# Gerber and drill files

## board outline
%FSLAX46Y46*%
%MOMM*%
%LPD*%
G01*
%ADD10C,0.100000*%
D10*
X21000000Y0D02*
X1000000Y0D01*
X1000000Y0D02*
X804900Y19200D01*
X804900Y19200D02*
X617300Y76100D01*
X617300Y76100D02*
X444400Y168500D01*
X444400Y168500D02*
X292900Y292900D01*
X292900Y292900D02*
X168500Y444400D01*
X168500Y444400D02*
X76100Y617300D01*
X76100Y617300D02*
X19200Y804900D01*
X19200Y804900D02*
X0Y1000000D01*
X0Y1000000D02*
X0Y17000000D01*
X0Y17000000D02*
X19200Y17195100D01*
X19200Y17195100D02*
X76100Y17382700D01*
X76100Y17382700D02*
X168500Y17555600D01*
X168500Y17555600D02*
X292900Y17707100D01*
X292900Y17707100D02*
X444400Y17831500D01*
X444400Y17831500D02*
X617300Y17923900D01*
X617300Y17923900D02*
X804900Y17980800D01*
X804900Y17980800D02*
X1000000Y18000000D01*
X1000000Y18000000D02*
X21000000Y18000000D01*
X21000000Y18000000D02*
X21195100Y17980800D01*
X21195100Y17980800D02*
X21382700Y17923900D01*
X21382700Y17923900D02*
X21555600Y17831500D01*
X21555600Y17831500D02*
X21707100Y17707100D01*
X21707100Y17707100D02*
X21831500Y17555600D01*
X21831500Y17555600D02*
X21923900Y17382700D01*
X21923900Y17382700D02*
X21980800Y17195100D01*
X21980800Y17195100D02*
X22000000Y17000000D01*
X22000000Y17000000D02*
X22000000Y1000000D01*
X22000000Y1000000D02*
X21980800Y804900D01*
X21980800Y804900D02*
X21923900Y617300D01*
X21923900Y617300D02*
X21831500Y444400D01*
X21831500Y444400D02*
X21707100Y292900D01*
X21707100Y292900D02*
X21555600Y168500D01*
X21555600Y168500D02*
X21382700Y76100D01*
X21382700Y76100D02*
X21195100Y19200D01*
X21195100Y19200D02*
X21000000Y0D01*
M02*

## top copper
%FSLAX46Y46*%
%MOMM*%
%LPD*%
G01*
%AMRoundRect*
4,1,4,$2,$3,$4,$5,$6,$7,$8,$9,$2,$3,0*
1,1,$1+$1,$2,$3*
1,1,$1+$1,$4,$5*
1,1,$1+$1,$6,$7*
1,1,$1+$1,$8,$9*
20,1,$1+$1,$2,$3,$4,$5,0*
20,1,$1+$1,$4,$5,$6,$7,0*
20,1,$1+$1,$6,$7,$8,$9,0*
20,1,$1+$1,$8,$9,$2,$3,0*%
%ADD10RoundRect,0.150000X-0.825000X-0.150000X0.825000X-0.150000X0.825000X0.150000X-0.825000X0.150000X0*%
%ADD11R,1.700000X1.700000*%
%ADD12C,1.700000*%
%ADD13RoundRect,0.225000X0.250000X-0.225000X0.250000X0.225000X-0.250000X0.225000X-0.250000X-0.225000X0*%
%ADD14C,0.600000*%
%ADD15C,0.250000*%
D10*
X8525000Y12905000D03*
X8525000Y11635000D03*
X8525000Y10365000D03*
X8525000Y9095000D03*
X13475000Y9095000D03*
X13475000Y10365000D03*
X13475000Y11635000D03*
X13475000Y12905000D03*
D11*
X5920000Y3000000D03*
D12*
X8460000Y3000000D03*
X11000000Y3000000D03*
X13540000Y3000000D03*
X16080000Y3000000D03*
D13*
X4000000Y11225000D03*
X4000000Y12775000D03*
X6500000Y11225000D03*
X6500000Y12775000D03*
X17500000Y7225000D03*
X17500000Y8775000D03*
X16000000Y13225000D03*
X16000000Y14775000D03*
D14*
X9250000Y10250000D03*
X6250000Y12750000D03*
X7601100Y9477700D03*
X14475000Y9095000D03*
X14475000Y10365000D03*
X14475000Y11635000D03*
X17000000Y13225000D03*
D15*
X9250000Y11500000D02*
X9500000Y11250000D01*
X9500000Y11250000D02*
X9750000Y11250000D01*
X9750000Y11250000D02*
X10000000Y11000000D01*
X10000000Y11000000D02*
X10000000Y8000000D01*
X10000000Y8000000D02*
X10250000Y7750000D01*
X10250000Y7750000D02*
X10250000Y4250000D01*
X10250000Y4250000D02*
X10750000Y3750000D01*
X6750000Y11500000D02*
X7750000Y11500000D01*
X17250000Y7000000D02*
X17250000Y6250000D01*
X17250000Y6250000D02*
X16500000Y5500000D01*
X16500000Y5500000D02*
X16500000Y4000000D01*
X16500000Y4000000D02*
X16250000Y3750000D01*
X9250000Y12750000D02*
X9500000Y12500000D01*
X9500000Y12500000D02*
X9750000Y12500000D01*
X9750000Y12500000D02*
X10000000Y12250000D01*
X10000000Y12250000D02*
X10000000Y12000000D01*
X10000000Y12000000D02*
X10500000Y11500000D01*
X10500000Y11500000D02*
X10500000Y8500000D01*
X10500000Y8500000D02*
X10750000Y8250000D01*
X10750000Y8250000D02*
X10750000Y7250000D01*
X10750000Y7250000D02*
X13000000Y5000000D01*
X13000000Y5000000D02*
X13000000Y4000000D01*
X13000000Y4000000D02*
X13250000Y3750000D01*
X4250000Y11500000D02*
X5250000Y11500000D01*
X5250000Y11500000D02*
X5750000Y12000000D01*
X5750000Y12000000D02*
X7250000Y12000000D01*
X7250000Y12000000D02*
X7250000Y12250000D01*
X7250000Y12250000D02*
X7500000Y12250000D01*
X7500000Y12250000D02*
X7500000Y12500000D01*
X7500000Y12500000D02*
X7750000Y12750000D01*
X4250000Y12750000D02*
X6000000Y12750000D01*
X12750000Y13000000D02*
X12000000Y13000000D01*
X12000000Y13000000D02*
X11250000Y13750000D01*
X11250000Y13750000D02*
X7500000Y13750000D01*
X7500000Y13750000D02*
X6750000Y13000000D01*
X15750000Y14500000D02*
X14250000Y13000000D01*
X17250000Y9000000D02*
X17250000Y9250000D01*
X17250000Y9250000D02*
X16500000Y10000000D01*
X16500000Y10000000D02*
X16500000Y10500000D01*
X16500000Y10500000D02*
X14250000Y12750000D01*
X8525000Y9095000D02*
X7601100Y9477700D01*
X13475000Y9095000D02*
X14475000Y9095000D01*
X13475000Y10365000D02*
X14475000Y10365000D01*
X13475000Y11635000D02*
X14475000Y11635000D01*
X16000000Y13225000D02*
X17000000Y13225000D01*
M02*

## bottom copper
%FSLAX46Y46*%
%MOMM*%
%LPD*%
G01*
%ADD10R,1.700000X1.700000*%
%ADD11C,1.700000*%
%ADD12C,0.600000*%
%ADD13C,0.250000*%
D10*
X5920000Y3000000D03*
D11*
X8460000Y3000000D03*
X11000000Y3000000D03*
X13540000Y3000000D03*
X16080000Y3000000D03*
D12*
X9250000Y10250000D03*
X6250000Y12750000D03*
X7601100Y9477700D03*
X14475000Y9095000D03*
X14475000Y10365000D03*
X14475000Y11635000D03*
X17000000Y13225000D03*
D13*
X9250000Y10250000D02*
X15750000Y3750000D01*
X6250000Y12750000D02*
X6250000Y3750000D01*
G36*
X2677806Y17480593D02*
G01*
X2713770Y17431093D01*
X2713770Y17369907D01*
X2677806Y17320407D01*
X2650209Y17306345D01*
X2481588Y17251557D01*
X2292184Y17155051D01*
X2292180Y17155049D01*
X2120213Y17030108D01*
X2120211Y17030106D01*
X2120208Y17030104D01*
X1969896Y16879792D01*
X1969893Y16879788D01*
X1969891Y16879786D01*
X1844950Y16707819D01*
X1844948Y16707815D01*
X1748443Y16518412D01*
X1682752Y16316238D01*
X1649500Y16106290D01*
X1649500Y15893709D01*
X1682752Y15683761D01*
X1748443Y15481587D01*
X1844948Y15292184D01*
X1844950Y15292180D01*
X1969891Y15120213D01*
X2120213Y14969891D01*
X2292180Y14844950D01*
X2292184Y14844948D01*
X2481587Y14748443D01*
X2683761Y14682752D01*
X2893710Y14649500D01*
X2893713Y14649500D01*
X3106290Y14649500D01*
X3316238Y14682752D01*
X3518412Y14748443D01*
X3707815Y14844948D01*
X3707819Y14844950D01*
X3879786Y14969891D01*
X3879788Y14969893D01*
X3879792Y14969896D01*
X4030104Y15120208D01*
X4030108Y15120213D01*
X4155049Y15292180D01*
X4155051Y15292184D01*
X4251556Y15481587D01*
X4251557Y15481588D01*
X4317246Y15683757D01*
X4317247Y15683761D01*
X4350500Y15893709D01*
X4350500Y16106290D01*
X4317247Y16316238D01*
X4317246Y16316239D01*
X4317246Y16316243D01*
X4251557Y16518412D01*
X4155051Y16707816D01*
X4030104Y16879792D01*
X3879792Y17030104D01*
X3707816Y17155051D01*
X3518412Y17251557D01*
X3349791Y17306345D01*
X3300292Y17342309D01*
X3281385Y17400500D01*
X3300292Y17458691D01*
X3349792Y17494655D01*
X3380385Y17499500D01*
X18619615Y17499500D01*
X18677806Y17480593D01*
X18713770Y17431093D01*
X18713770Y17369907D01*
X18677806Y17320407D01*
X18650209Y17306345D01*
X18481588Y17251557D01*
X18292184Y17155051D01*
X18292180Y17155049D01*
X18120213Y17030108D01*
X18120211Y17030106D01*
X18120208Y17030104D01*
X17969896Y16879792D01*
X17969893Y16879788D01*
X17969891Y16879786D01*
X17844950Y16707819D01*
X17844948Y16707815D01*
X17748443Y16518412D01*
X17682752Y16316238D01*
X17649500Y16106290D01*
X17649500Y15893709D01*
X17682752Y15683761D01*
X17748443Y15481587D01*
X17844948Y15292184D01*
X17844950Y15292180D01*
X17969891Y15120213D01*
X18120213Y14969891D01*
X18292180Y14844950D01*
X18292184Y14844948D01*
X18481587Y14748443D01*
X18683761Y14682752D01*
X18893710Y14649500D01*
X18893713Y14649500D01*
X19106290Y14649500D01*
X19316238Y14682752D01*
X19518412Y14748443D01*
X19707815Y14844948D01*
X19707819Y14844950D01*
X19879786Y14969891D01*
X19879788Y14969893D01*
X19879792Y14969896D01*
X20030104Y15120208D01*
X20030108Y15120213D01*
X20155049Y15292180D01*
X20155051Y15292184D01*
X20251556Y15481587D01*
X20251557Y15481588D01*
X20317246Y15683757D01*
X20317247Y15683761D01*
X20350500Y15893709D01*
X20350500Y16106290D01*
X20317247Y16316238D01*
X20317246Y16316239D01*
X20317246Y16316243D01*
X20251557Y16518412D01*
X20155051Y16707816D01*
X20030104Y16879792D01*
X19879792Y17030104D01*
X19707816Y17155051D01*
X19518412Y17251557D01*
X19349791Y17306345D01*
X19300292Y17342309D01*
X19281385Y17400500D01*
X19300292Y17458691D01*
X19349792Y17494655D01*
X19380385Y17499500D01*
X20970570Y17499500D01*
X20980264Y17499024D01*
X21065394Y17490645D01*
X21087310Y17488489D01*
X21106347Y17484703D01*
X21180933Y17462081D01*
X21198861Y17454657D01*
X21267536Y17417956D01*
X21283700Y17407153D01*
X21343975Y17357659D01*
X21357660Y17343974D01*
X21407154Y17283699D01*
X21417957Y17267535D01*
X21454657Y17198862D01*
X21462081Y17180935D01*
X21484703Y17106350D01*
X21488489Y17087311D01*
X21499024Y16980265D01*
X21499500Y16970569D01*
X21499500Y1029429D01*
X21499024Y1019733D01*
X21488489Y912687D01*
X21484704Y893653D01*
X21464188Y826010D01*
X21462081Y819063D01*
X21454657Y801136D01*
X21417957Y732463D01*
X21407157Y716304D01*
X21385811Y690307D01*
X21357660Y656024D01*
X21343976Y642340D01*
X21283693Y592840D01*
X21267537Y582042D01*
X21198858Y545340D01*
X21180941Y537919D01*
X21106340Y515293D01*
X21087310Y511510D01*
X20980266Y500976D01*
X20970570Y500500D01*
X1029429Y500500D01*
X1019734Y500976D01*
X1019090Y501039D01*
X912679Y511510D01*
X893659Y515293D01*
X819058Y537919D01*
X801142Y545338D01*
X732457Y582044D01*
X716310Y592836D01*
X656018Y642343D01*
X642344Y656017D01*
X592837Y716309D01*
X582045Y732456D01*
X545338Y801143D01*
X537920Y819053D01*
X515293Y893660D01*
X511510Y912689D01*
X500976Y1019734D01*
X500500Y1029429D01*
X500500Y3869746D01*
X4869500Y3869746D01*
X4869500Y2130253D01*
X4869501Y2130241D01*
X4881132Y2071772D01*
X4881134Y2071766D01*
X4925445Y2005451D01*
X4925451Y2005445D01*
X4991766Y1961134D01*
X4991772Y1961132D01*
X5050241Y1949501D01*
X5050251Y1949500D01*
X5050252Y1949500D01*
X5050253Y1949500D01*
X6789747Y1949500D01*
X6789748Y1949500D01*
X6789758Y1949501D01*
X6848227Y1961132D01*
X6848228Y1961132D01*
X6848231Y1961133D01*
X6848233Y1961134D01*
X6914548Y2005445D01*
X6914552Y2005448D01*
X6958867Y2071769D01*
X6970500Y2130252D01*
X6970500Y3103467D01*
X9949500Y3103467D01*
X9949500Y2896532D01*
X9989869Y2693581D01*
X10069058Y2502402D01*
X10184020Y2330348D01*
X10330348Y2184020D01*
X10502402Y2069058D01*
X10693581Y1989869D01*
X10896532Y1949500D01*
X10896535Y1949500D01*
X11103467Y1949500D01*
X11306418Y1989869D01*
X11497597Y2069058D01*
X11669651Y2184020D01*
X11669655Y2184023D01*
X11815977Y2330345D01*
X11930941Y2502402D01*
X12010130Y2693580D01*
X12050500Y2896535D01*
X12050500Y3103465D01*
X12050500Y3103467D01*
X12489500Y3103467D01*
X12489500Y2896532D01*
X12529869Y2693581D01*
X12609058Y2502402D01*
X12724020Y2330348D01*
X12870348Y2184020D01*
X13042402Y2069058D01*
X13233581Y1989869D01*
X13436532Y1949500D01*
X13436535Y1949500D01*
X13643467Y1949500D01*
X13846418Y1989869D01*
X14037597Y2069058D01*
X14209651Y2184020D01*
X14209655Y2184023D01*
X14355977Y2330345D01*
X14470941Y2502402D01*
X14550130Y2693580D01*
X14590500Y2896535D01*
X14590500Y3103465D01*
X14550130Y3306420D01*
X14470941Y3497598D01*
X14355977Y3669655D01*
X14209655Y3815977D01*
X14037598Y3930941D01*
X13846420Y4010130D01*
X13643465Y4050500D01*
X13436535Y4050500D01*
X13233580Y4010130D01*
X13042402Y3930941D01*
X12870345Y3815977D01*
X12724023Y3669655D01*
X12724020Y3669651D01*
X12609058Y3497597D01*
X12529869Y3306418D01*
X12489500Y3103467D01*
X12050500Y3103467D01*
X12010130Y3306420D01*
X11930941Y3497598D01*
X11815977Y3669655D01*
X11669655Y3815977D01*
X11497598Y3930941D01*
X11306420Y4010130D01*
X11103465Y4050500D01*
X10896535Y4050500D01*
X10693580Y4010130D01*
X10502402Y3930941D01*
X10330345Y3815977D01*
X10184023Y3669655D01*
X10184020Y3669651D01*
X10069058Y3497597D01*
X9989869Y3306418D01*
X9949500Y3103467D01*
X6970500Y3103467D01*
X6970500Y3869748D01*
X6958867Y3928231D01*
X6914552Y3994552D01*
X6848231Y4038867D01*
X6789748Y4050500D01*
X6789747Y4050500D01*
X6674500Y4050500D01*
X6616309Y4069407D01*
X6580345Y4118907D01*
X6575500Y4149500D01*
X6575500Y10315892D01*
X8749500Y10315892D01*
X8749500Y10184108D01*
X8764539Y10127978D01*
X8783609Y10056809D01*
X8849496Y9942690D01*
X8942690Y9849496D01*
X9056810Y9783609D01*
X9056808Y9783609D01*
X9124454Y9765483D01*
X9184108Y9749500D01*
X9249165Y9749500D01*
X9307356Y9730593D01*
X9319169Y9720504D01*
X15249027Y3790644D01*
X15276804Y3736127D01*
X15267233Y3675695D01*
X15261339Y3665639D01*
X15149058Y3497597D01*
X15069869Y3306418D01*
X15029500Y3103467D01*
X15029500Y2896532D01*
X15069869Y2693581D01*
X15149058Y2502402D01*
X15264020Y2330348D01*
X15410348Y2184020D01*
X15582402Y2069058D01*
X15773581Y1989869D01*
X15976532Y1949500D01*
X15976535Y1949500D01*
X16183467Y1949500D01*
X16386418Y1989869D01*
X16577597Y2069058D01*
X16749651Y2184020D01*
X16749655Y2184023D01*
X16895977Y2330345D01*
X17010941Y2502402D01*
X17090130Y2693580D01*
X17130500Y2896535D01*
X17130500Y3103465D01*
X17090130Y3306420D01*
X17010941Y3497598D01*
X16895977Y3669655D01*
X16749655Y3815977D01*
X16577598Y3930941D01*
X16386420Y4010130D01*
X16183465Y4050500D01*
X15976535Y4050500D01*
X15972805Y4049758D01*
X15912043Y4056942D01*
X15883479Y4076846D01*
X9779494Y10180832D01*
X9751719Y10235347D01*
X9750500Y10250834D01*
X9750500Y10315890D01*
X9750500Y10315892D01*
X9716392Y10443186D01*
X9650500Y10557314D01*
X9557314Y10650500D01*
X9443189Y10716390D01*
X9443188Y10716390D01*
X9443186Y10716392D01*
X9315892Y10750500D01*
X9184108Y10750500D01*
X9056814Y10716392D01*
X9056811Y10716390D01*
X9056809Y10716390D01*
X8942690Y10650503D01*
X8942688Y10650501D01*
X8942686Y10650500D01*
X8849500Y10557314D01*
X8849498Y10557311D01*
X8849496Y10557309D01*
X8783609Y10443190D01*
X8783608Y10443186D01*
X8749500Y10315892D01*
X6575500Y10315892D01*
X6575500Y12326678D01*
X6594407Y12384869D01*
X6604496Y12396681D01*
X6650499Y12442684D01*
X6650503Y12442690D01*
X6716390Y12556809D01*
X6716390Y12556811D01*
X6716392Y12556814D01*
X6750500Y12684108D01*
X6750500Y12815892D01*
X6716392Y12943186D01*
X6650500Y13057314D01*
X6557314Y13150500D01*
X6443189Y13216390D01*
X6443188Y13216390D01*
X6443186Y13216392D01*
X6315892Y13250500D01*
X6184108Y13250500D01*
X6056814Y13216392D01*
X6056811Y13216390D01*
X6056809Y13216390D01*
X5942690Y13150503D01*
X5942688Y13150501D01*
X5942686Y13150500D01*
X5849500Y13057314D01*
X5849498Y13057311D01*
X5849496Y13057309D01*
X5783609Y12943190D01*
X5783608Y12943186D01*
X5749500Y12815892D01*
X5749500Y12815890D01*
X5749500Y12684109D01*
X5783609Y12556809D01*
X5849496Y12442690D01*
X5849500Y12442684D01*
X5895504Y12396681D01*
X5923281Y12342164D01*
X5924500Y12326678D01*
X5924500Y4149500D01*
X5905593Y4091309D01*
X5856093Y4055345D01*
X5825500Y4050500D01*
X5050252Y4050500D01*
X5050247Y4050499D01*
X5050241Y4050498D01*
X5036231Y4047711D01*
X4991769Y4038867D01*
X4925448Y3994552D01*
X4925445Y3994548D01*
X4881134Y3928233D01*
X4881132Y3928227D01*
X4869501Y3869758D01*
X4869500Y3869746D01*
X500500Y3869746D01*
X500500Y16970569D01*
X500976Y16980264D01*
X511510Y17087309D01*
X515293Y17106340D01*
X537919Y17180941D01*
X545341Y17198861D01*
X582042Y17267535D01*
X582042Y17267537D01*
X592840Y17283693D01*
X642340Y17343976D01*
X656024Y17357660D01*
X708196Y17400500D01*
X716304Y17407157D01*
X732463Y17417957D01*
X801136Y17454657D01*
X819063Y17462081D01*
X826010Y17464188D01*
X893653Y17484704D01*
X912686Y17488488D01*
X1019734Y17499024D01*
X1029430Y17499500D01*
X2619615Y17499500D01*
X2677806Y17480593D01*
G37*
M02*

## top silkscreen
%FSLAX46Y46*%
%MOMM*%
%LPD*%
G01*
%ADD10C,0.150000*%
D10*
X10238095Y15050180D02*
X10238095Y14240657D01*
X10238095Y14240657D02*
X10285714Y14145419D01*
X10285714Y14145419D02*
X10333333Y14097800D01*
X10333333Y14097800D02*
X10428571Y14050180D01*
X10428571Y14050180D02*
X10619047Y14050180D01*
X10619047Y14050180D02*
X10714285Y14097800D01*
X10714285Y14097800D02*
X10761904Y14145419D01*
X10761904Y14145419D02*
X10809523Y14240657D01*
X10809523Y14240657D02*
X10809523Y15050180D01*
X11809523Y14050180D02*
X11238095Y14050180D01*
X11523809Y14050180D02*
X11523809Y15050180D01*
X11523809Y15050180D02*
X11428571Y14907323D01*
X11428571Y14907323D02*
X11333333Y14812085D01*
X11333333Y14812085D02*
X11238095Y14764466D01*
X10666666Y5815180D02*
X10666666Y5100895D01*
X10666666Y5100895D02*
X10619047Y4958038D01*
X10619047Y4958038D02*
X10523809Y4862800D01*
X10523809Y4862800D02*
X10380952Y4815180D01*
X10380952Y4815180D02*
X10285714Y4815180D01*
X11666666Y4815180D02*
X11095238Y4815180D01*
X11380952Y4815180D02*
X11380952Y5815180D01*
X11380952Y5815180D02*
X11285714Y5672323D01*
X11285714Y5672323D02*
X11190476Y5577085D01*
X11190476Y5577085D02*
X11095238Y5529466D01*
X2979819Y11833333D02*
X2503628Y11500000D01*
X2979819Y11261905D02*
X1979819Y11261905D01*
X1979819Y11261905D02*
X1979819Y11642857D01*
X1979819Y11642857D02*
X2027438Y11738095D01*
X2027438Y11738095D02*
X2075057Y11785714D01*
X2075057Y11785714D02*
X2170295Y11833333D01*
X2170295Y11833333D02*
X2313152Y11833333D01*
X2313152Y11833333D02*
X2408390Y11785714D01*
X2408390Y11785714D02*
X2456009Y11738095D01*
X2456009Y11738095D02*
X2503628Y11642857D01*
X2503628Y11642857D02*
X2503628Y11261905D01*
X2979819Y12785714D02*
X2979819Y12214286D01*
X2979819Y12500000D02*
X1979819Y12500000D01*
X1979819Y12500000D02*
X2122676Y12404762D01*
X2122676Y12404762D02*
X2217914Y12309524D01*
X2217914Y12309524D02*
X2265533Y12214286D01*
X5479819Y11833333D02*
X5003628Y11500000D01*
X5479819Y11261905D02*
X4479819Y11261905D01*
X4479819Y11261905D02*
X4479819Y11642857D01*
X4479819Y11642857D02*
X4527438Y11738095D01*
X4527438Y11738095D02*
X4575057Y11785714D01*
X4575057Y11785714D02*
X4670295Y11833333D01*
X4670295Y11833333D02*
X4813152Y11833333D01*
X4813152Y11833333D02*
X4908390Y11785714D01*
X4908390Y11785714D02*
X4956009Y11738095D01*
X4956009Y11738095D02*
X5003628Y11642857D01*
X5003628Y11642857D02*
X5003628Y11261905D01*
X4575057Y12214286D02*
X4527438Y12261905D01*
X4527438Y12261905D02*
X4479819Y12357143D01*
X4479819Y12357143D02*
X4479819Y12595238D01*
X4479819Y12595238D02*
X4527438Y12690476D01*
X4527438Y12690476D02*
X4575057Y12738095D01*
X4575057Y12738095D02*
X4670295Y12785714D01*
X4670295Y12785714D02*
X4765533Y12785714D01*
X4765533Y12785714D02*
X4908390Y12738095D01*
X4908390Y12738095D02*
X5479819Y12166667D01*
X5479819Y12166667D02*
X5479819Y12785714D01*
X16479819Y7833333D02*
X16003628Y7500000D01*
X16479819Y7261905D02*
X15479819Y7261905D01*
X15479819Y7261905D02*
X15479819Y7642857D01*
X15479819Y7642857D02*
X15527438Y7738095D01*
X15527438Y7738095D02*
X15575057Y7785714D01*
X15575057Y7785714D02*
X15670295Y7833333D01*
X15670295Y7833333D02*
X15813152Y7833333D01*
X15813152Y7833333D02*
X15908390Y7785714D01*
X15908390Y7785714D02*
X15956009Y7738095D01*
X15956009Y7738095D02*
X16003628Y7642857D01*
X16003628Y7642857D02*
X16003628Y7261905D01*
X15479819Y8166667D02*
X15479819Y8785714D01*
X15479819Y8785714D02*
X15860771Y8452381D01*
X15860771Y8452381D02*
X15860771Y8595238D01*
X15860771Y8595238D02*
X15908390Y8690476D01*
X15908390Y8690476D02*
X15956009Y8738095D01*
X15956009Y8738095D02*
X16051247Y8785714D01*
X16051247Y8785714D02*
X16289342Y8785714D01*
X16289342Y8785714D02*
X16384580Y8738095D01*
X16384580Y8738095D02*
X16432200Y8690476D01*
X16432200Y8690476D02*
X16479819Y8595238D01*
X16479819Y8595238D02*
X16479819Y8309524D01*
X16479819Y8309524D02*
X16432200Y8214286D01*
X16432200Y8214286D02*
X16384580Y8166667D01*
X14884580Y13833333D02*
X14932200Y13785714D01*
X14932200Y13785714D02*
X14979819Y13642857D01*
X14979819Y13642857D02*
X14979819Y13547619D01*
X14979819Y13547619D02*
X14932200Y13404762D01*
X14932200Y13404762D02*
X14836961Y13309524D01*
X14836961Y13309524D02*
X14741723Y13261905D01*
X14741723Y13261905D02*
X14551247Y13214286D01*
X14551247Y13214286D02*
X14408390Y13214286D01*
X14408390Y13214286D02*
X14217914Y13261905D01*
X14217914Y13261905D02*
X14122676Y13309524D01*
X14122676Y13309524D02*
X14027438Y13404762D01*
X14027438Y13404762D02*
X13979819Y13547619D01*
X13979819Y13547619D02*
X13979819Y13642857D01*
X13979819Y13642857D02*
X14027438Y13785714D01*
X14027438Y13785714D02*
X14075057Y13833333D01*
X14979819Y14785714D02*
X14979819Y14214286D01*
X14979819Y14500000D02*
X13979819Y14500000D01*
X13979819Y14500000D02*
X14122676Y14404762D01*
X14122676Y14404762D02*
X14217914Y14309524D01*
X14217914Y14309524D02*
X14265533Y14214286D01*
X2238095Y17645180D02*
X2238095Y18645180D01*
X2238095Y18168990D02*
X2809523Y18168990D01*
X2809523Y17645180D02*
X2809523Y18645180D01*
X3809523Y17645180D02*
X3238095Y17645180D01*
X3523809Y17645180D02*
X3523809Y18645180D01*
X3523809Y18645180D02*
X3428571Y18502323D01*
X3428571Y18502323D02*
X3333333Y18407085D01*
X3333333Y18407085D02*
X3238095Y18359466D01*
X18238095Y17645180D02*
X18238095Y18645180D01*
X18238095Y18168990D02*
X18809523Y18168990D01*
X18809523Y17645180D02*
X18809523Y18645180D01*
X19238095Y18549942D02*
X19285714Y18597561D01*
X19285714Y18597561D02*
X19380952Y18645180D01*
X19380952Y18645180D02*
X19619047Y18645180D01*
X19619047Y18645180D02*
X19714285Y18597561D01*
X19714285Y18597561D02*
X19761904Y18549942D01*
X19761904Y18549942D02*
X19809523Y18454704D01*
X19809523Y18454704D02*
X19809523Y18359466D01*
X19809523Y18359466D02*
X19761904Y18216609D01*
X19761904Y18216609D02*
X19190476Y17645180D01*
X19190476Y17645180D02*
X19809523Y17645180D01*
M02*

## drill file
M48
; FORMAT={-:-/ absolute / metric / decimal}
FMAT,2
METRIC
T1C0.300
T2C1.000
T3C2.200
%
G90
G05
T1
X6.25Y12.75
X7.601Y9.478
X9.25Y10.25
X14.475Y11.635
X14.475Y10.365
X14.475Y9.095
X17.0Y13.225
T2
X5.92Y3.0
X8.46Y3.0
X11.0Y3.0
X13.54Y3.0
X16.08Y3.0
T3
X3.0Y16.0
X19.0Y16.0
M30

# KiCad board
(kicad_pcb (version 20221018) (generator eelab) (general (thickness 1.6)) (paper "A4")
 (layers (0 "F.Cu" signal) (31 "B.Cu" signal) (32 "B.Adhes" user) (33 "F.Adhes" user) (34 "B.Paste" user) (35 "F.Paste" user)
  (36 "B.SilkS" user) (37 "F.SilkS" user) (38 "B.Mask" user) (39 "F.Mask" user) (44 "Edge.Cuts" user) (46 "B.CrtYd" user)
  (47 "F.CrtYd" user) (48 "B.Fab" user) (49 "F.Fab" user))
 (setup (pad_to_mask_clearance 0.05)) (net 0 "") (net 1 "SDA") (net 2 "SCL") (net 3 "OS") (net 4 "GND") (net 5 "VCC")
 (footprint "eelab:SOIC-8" (layer "F.Cu") (at 11.0000 -11.0000 0)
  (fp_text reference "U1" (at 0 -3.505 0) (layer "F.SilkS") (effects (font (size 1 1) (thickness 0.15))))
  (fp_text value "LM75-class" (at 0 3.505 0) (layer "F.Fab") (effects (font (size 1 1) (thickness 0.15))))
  (pad "1" smd roundrect (at -2.4750 -1.9050 0) (size 1.9500 0.6000) (layers "F.Cu" "F.Paste" "F.Mask") (roundrect_rratio 0.25)
   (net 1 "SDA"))
  (pad "2" smd roundrect (at -2.4750 -0.6350 0) (size 1.9500 0.6000) (layers "F.Cu" "F.Paste" "F.Mask") (roundrect_rratio 0.25)
   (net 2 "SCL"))
  (pad "3" smd roundrect (at -2.4750 0.6350 0) (size 1.9500 0.6000) (layers "F.Cu" "F.Paste" "F.Mask") (roundrect_rratio 0.25) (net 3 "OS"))
  (pad "4" smd roundrect (at -2.4750 1.9050 0) (size 1.9500 0.6000) (layers "F.Cu" "F.Paste" "F.Mask") (roundrect_rratio 0.25) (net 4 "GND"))
  (pad "5" smd roundrect (at 2.4750 1.9050 0) (size 1.9500 0.6000) (layers "F.Cu" "F.Paste" "F.Mask") (roundrect_rratio 0.25) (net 4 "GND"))
  (pad "6" smd roundrect (at 2.4750 0.6350 0) (size 1.9500 0.6000) (layers "F.Cu" "F.Paste" "F.Mask") (roundrect_rratio 0.25) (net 4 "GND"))
  (pad "7" smd roundrect (at 2.4750 -0.6350 0) (size 1.9500 0.6000) (layers "F.Cu" "F.Paste" "F.Mask") (roundrect_rratio 0.25) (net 4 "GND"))
  (pad "8" smd roundrect (at 2.4750 -1.9050 0) (size 1.9500 0.6000) (layers "F.Cu" "F.Paste" "F.Mask") (roundrect_rratio 0.25) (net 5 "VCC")))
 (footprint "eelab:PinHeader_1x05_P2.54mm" (layer "F.Cu") (at 11.0000 -3.0000 0)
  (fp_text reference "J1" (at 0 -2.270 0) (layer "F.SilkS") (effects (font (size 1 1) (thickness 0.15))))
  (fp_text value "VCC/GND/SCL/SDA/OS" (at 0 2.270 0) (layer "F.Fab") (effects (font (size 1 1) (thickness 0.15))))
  (pad "1" thru_hole rect (at -5.0800 -0.0000 0) (size 1.7000 1.7000) (drill 1.0) (layers "*.Cu" "*.Mask") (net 5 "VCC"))
  (pad "2" thru_hole circle (at -2.5400 -0.0000 0) (size 1.7000 1.7000) (drill 1.0) (layers "*.Cu" "*.Mask") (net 4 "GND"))
  (pad "3" thru_hole circle (at 0.0000 -0.0000 0) (size 1.7000 1.7000) (drill 1.0) (layers "*.Cu" "*.Mask") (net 2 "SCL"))
  (pad "4" thru_hole circle (at 2.5400 -0.0000 0) (size 1.7000 1.7000) (drill 1.0) (layers "*.Cu" "*.Mask") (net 1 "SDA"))
  (pad "5" thru_hole circle (at 5.0800 -0.0000 0) (size 1.7000 1.7000) (drill 1.0) (layers "*.Cu" "*.Mask") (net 3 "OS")))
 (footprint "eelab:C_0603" (layer "F.Cu") (at 4.0000 -12.0000 90)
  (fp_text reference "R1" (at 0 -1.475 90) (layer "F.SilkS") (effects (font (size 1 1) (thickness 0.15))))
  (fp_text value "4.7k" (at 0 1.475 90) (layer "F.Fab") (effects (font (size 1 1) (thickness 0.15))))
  (pad "1" smd roundrect (at -0.7750 0.0000 90) (size 0.9000 0.9500) (layers "F.Cu" "F.Paste" "F.Mask") (roundrect_rratio 0.25)
   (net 1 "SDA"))
  (pad "2" smd roundrect (at 0.7750 0.0000 90) (size 0.9000 0.9500) (layers "F.Cu" "F.Paste" "F.Mask") (roundrect_rratio 0.25) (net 5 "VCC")))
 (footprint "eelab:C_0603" (layer "F.Cu") (at 6.5000 -12.0000 90)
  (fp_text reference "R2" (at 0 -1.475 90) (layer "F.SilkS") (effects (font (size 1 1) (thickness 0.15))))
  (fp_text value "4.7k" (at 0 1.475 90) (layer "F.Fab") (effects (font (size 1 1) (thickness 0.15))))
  (pad "1" smd roundrect (at -0.7750 0.0000 90) (size 0.9000 0.9500) (layers "F.Cu" "F.Paste" "F.Mask") (roundrect_rratio 0.25)
   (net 2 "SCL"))
  (pad "2" smd roundrect (at 0.7750 0.0000 90) (size 0.9000 0.9500) (layers "F.Cu" "F.Paste" "F.Mask") (roundrect_rratio 0.25) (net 5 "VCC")))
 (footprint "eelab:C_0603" (layer "F.Cu") (at 17.5000 -8.0000 90)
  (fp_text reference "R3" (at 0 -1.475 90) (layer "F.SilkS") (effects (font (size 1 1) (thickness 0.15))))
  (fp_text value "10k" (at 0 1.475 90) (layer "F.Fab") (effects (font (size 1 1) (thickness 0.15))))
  (pad "1" smd roundrect (at -0.7750 0.0000 90) (size 0.9000 0.9500) (layers "F.Cu" "F.Paste" "F.Mask") (roundrect_rratio 0.25) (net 3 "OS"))
  (pad "2" smd roundrect (at 0.7750 0.0000 90) (size 0.9000 0.9500) (layers "F.Cu" "F.Paste" "F.Mask") (roundrect_rratio 0.25) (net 5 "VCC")))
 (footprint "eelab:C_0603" (layer "F.Cu") (at 16.0000 -14.0000 90)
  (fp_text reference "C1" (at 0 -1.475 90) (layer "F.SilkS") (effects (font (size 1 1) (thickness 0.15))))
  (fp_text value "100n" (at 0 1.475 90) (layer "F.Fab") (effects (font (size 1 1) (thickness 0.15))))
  (pad "1" smd roundrect (at -0.7750 0.0000 90) (size 0.9000 0.9500) (layers "F.Cu" "F.Paste" "F.Mask") (roundrect_rratio 0.25)
   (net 4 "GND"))
  (pad "2" smd roundrect (at 0.7750 0.0000 90) (size 0.9000 0.9500) (layers "F.Cu" "F.Paste" "F.Mask") (roundrect_rratio 0.25) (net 5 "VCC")))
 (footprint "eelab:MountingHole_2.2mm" (layer "F.Cu") (at 3.0000 -16.0000 0)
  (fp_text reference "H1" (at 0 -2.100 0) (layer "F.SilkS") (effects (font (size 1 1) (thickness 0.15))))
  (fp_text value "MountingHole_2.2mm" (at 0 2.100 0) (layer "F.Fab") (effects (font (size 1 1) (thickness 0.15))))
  (pad "" np_thru_hole circle (at 0.0000 0.0000 0) (size 2.2000 2.2000) (drill 2.2) (layers "*.Cu" "*.Mask")))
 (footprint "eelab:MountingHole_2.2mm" (layer "F.Cu") (at 19.0000 -16.0000 0)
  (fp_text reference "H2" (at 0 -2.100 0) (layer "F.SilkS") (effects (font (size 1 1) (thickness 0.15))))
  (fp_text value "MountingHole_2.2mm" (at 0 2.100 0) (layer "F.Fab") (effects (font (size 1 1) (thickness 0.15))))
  (pad "" np_thru_hole circle (at 0.0000 0.0000 0) (size 2.2000 2.2000) (drill 2.2) (layers "*.Cu" "*.Mask")))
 (gr_line (start 21.0000 -0.0000) (end 1.0000 -0.0000) (stroke (width 0.1) (type solid)) (layer "Edge.Cuts"))
 (gr_line (start 1.0000 -0.0000) (end 0.8049 -0.0192) (stroke (width 0.1) (type solid)) (layer "Edge.Cuts"))
 (gr_line (start 0.8049 -0.0192) (end 0.6173 -0.0761) (stroke (width 0.1) (type solid)) (layer "Edge.Cuts"))
 (gr_line (start 0.6173 -0.0761) (end 0.4444 -0.1685) (stroke (width 0.1) (type solid)) (layer "Edge.Cuts"))
 (gr_line (start 0.4444 -0.1685) (end 0.2929 -0.2929) (stroke (width 0.1) (type solid)) (layer "Edge.Cuts"))
 (gr_line (start 0.2929 -0.2929) (end 0.1685 -0.4444) (stroke (width 0.1) (type solid)) (layer "Edge.Cuts"))
 (gr_line (start 0.1685 -0.4444) (end 0.0761 -0.6173) (stroke (width 0.1) (type solid)) (layer "Edge.Cuts"))
 (gr_line (start 0.0761 -0.6173) (end 0.0192 -0.8049) (stroke (width 0.1) (type solid)) (layer "Edge.Cuts"))
 (gr_line (start 0.0192 -0.8049) (end 0.0000 -1.0000) (stroke (width 0.1) (type solid)) (layer "Edge.Cuts"))
 (gr_line (start 0.0000 -1.0000) (end 0.0000 -17.0000) (stroke (width 0.1) (type solid)) (layer "Edge.Cuts"))
 (gr_line (start 0.0000 -17.0000) (end 0.0192 -17.1951) (stroke (width 0.1) (type solid)) (layer "Edge.Cuts"))
 (gr_line (start 0.0192 -17.1951) (end 0.0761 -17.3827) (stroke (width 0.1) (type solid)) (layer "Edge.Cuts"))
 (gr_line (start 0.0761 -17.3827) (end 0.1685 -17.5556) (stroke (width 0.1) (type solid)) (layer "Edge.Cuts"))
 (gr_line (start 0.1685 -17.5556) (end 0.2929 -17.7071) (stroke (width 0.1) (type solid)) (layer "Edge.Cuts"))
 (gr_line (start 0.2929 -17.7071) (end 0.4444 -17.8315) (stroke (width 0.1) (type solid)) (layer "Edge.Cuts"))
 (gr_line (start 0.4444 -17.8315) (end 0.6173 -17.9239) (stroke (width 0.1) (type solid)) (layer "Edge.Cuts"))
 (gr_line (start 0.6173 -17.9239) (end 0.8049 -17.9808) (stroke (width 0.1) (type solid)) (layer "Edge.Cuts"))
 (gr_line (start 0.8049 -17.9808) (end 1.0000 -18.0000) (stroke (width 0.1) (type solid)) (layer "Edge.Cuts"))
 (gr_line (start 1.0000 -18.0000) (end 21.0000 -18.0000) (stroke (width 0.1) (type solid)) (layer "Edge.Cuts"))
 (gr_line (start 21.0000 -18.0000) (end 21.1951 -17.9808) (stroke (width 0.1) (type solid)) (layer "Edge.Cuts"))
 (gr_line (start 21.1951 -17.9808) (end 21.3827 -17.9239) (stroke (width 0.1) (type solid)) (layer "Edge.Cuts"))
 (gr_line (start 21.3827 -17.9239) (end 21.5556 -17.8315) (stroke (width 0.1) (type solid)) (layer "Edge.Cuts"))
 (gr_line (start 21.5556 -17.8315) (end 21.7071 -17.7071) (stroke (width 0.1) (type solid)) (layer "Edge.Cuts"))
 (gr_line (start 21.7071 -17.7071) (end 21.8315 -17.5556) (stroke (width 0.1) (type solid)) (layer "Edge.Cuts"))
 (gr_line (start 21.8315 -17.5556) (end 21.9239 -17.3827) (stroke (width 0.1) (type solid)) (layer "Edge.Cuts"))
 (gr_line (start 21.9239 -17.3827) (end 21.9808 -17.1951) (stroke (width 0.1) (type solid)) (layer "Edge.Cuts"))
 (gr_line (start 21.9808 -17.1951) (end 22.0000 -17.0000) (stroke (width 0.1) (type solid)) (layer "Edge.Cuts"))
 (gr_line (start 22.0000 -17.0000) (end 22.0000 -1.0000) (stroke (width 0.1) (type solid)) (layer "Edge.Cuts"))
 (gr_line (start 22.0000 -1.0000) (end 21.9808 -0.8049) (stroke (width 0.1) (type solid)) (layer "Edge.Cuts"))
 (gr_line (start 21.9808 -0.8049) (end 21.9239 -0.6173) (stroke (width 0.1) (type solid)) (layer "Edge.Cuts"))
 (gr_line (start 21.9239 -0.6173) (end 21.8315 -0.4444) (stroke (width 0.1) (type solid)) (layer "Edge.Cuts"))
 (gr_line (start 21.8315 -0.4444) (end 21.7071 -0.2929) (stroke (width 0.1) (type solid)) (layer "Edge.Cuts"))
 (gr_line (start 21.7071 -0.2929) (end 21.5556 -0.1685) (stroke (width 0.1) (type solid)) (layer "Edge.Cuts"))
 (gr_line (start 21.5556 -0.1685) (end 21.3827 -0.0761) (stroke (width 0.1) (type solid)) (layer "Edge.Cuts"))
 (gr_line (start 21.3827 -0.0761) (end 21.1951 -0.0192) (stroke (width 0.1) (type solid)) (layer "Edge.Cuts"))
 (gr_line (start 21.1951 -0.0192) (end 21.0000 -0.0000) (stroke (width 0.1) (type solid)) (layer "Edge.Cuts"))
 (segment (start 9.2500 -11.5000) (end 9.5000 -11.2500) (width 0.25) (layer "F.Cu") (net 2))
 (segment (start 9.5000 -11.2500) (end 9.7500 -11.2500) (width 0.25) (layer "F.Cu") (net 2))
 (segment (start 9.7500 -11.2500) (end 10.0000 -11.0000) (width 0.25) (layer "F.Cu") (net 2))
 (segment (start 10.0000 -11.0000) (end 10.0000 -8.0000) (width 0.25) (layer "F.Cu") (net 2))
 (segment (start 10.0000 -8.0000) (end 10.2500 -7.7500) (width 0.25) (layer "F.Cu") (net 2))
 (segment (start 10.2500 -7.7500) (end 10.2500 -4.2500) (width 0.25) (layer "F.Cu") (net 2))
 (segment (start 10.2500 -4.2500) (end 10.7500 -3.7500) (width 0.25) (layer "F.Cu") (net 2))
 (segment (start 6.7500 -11.5000) (end 7.7500 -11.5000) (width 0.25) (layer "F.Cu") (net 2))
 (segment (start 17.2500 -7.0000) (end 17.2500 -6.2500) (width 0.25) (layer "F.Cu") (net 3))
 (segment (start 17.2500 -6.2500) (end 16.5000 -5.5000) (width 0.25) (layer "F.Cu") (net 3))
 (segment (start 16.5000 -5.5000) (end 16.5000 -4.0000) (width 0.25) (layer "F.Cu") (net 3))
 (segment (start 16.5000 -4.0000) (end 16.2500 -3.7500) (width 0.25) (layer "F.Cu") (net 3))
 (segment (start 9.2500 -10.2500) (end 15.7500 -3.7500) (width 0.25) (layer "B.Cu") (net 3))
 (segment (start 9.2500 -12.7500) (end 9.5000 -12.5000) (width 0.25) (layer "F.Cu") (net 1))
 (segment (start 9.5000 -12.5000) (end 9.7500 -12.5000) (width 0.25) (layer "F.Cu") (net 1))
 (segment (start 9.7500 -12.5000) (end 10.0000 -12.2500) (width 0.25) (layer "F.Cu") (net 1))
 (segment (start 10.0000 -12.2500) (end 10.0000 -12.0000) (width 0.25) (layer "F.Cu") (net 1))
 (segment (start 10.0000 -12.0000) (end 10.5000 -11.5000) (width 0.25) (layer "F.Cu") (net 1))
 (segment (start 10.5000 -11.5000) (end 10.5000 -8.5000) (width 0.25) (layer "F.Cu") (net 1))
 (segment (start 10.5000 -8.5000) (end 10.7500 -8.2500) (width 0.25) (layer "F.Cu") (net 1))
 (segment (start 10.7500 -8.2500) (end 10.7500 -7.2500) (width 0.25) (layer "F.Cu") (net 1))
 (segment (start 10.7500 -7.2500) (end 13.0000 -5.0000) (width 0.25) (layer "F.Cu") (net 1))
 (segment (start 13.0000 -5.0000) (end 13.0000 -4.0000) (width 0.25) (layer "F.Cu") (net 1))
 (segment (start 13.0000 -4.0000) (end 13.2500 -3.7500) (width 0.25) (layer "F.Cu") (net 1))
 (segment (start 4.2500 -11.5000) (end 5.2500 -11.5000) (width 0.25) (layer "F.Cu") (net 1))
 (segment (start 5.2500 -11.5000) (end 5.7500 -12.0000) (width 0.25) (layer "F.Cu") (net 1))
 (segment (start 5.7500 -12.0000) (end 7.2500 -12.0000) (width 0.25) (layer "F.Cu") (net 1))
 (segment (start 7.2500 -12.0000) (end 7.2500 -12.2500) (width 0.25) (layer "F.Cu") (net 1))
 (segment (start 7.2500 -12.2500) (end 7.5000 -12.2500) (width 0.25) (layer "F.Cu") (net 1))
 (segment (start 7.5000 -12.2500) (end 7.5000 -12.5000) (width 0.25) (layer "F.Cu") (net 1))
 (segment (start 7.5000 -12.5000) (end 7.7500 -12.7500) (width 0.25) (layer "F.Cu") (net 1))
 (segment (start 6.2500 -12.7500) (end 6.2500 -3.7500) (width 0.25) (layer "B.Cu") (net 5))
 (segment (start 4.2500 -12.7500) (end 6.0000 -12.7500) (width 0.25) (layer "F.Cu") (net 5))
 (segment (start 12.7500 -13.0000) (end 12.0000 -13.0000) (width 0.25) (layer "F.Cu") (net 5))
 (segment (start 12.0000 -13.0000) (end 11.2500 -13.7500) (width 0.25) (layer "F.Cu") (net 5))
 (segment (start 11.2500 -13.7500) (end 7.5000 -13.7500) (width 0.25) (layer "F.Cu") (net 5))
 (segment (start 7.5000 -13.7500) (end 6.7500 -13.0000) (width 0.25) (layer "F.Cu") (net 5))
 (segment (start 15.7500 -14.5000) (end 14.2500 -13.0000) (width 0.25) (layer "F.Cu") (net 5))
 (segment (start 17.2500 -9.0000) (end 17.2500 -9.2500) (width 0.25) (layer "F.Cu") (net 5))
 (segment (start 17.2500 -9.2500) (end 16.5000 -10.0000) (width 0.25) (layer "F.Cu") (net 5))
 (segment (start 16.5000 -10.0000) (end 16.5000 -10.5000) (width 0.25) (layer "F.Cu") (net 5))
 (segment (start 16.5000 -10.5000) (end 14.2500 -12.7500) (width 0.25) (layer "F.Cu") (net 5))
 (segment (start 8.5250 -9.0950) (end 7.6011 -9.4777) (width 0.25) (layer "F.Cu") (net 4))
 (segment (start 13.4750 -9.0950) (end 14.4750 -9.0950) (width 0.25) (layer "F.Cu") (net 4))
 (segment (start 13.4750 -10.3650) (end 14.4750 -10.3650) (width 0.25) (layer "F.Cu") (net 4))
 (segment (start 13.4750 -11.6350) (end 14.4750 -11.6350) (width 0.25) (layer "F.Cu") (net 4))
 (segment (start 16.0000 -13.2250) (end 17.0000 -13.2250) (width 0.25) (layer "F.Cu") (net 4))
 (via (at 9.2500 -10.2500) (size 0.6) (drill 0.3) (layers "F.Cu" "B.Cu") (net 3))
 (via (at 6.2500 -12.7500) (size 0.6) (drill 0.3) (layers "F.Cu" "B.Cu") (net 5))
 (via (at 7.6011 -9.4777) (size 0.6) (drill 0.3) (layers "F.Cu" "B.Cu") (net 4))
 (via (at 14.4750 -9.0950) (size 0.6) (drill 0.3) (layers "F.Cu" "B.Cu") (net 4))
 (via (at 14.4750 -10.3650) (size 0.6) (drill 0.3) (layers "F.Cu" "B.Cu") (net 4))
 (via (at 14.4750 -11.6350) (size 0.6) (drill 0.3) (layers "F.Cu" "B.Cu") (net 4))
 (via (at 17.0000 -13.2250) (size 0.6) (drill 0.3) (layers "F.Cu" "B.Cu") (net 4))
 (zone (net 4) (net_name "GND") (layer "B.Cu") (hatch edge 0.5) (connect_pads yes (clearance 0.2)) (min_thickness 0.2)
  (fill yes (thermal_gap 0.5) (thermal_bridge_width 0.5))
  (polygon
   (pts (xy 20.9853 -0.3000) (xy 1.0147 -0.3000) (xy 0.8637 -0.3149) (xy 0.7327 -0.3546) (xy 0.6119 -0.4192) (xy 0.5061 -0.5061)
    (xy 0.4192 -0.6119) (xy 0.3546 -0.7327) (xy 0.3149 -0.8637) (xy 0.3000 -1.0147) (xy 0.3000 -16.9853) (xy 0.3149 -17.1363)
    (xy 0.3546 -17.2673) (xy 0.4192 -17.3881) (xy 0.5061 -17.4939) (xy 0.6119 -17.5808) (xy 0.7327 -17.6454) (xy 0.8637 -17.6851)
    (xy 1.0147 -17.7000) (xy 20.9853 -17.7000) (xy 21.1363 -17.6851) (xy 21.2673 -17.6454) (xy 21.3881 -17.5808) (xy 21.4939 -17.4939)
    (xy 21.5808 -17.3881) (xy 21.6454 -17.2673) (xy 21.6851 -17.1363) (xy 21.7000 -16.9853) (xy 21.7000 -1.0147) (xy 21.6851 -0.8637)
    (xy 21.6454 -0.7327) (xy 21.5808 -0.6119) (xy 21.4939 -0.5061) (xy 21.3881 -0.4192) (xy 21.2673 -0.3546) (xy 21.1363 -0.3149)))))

